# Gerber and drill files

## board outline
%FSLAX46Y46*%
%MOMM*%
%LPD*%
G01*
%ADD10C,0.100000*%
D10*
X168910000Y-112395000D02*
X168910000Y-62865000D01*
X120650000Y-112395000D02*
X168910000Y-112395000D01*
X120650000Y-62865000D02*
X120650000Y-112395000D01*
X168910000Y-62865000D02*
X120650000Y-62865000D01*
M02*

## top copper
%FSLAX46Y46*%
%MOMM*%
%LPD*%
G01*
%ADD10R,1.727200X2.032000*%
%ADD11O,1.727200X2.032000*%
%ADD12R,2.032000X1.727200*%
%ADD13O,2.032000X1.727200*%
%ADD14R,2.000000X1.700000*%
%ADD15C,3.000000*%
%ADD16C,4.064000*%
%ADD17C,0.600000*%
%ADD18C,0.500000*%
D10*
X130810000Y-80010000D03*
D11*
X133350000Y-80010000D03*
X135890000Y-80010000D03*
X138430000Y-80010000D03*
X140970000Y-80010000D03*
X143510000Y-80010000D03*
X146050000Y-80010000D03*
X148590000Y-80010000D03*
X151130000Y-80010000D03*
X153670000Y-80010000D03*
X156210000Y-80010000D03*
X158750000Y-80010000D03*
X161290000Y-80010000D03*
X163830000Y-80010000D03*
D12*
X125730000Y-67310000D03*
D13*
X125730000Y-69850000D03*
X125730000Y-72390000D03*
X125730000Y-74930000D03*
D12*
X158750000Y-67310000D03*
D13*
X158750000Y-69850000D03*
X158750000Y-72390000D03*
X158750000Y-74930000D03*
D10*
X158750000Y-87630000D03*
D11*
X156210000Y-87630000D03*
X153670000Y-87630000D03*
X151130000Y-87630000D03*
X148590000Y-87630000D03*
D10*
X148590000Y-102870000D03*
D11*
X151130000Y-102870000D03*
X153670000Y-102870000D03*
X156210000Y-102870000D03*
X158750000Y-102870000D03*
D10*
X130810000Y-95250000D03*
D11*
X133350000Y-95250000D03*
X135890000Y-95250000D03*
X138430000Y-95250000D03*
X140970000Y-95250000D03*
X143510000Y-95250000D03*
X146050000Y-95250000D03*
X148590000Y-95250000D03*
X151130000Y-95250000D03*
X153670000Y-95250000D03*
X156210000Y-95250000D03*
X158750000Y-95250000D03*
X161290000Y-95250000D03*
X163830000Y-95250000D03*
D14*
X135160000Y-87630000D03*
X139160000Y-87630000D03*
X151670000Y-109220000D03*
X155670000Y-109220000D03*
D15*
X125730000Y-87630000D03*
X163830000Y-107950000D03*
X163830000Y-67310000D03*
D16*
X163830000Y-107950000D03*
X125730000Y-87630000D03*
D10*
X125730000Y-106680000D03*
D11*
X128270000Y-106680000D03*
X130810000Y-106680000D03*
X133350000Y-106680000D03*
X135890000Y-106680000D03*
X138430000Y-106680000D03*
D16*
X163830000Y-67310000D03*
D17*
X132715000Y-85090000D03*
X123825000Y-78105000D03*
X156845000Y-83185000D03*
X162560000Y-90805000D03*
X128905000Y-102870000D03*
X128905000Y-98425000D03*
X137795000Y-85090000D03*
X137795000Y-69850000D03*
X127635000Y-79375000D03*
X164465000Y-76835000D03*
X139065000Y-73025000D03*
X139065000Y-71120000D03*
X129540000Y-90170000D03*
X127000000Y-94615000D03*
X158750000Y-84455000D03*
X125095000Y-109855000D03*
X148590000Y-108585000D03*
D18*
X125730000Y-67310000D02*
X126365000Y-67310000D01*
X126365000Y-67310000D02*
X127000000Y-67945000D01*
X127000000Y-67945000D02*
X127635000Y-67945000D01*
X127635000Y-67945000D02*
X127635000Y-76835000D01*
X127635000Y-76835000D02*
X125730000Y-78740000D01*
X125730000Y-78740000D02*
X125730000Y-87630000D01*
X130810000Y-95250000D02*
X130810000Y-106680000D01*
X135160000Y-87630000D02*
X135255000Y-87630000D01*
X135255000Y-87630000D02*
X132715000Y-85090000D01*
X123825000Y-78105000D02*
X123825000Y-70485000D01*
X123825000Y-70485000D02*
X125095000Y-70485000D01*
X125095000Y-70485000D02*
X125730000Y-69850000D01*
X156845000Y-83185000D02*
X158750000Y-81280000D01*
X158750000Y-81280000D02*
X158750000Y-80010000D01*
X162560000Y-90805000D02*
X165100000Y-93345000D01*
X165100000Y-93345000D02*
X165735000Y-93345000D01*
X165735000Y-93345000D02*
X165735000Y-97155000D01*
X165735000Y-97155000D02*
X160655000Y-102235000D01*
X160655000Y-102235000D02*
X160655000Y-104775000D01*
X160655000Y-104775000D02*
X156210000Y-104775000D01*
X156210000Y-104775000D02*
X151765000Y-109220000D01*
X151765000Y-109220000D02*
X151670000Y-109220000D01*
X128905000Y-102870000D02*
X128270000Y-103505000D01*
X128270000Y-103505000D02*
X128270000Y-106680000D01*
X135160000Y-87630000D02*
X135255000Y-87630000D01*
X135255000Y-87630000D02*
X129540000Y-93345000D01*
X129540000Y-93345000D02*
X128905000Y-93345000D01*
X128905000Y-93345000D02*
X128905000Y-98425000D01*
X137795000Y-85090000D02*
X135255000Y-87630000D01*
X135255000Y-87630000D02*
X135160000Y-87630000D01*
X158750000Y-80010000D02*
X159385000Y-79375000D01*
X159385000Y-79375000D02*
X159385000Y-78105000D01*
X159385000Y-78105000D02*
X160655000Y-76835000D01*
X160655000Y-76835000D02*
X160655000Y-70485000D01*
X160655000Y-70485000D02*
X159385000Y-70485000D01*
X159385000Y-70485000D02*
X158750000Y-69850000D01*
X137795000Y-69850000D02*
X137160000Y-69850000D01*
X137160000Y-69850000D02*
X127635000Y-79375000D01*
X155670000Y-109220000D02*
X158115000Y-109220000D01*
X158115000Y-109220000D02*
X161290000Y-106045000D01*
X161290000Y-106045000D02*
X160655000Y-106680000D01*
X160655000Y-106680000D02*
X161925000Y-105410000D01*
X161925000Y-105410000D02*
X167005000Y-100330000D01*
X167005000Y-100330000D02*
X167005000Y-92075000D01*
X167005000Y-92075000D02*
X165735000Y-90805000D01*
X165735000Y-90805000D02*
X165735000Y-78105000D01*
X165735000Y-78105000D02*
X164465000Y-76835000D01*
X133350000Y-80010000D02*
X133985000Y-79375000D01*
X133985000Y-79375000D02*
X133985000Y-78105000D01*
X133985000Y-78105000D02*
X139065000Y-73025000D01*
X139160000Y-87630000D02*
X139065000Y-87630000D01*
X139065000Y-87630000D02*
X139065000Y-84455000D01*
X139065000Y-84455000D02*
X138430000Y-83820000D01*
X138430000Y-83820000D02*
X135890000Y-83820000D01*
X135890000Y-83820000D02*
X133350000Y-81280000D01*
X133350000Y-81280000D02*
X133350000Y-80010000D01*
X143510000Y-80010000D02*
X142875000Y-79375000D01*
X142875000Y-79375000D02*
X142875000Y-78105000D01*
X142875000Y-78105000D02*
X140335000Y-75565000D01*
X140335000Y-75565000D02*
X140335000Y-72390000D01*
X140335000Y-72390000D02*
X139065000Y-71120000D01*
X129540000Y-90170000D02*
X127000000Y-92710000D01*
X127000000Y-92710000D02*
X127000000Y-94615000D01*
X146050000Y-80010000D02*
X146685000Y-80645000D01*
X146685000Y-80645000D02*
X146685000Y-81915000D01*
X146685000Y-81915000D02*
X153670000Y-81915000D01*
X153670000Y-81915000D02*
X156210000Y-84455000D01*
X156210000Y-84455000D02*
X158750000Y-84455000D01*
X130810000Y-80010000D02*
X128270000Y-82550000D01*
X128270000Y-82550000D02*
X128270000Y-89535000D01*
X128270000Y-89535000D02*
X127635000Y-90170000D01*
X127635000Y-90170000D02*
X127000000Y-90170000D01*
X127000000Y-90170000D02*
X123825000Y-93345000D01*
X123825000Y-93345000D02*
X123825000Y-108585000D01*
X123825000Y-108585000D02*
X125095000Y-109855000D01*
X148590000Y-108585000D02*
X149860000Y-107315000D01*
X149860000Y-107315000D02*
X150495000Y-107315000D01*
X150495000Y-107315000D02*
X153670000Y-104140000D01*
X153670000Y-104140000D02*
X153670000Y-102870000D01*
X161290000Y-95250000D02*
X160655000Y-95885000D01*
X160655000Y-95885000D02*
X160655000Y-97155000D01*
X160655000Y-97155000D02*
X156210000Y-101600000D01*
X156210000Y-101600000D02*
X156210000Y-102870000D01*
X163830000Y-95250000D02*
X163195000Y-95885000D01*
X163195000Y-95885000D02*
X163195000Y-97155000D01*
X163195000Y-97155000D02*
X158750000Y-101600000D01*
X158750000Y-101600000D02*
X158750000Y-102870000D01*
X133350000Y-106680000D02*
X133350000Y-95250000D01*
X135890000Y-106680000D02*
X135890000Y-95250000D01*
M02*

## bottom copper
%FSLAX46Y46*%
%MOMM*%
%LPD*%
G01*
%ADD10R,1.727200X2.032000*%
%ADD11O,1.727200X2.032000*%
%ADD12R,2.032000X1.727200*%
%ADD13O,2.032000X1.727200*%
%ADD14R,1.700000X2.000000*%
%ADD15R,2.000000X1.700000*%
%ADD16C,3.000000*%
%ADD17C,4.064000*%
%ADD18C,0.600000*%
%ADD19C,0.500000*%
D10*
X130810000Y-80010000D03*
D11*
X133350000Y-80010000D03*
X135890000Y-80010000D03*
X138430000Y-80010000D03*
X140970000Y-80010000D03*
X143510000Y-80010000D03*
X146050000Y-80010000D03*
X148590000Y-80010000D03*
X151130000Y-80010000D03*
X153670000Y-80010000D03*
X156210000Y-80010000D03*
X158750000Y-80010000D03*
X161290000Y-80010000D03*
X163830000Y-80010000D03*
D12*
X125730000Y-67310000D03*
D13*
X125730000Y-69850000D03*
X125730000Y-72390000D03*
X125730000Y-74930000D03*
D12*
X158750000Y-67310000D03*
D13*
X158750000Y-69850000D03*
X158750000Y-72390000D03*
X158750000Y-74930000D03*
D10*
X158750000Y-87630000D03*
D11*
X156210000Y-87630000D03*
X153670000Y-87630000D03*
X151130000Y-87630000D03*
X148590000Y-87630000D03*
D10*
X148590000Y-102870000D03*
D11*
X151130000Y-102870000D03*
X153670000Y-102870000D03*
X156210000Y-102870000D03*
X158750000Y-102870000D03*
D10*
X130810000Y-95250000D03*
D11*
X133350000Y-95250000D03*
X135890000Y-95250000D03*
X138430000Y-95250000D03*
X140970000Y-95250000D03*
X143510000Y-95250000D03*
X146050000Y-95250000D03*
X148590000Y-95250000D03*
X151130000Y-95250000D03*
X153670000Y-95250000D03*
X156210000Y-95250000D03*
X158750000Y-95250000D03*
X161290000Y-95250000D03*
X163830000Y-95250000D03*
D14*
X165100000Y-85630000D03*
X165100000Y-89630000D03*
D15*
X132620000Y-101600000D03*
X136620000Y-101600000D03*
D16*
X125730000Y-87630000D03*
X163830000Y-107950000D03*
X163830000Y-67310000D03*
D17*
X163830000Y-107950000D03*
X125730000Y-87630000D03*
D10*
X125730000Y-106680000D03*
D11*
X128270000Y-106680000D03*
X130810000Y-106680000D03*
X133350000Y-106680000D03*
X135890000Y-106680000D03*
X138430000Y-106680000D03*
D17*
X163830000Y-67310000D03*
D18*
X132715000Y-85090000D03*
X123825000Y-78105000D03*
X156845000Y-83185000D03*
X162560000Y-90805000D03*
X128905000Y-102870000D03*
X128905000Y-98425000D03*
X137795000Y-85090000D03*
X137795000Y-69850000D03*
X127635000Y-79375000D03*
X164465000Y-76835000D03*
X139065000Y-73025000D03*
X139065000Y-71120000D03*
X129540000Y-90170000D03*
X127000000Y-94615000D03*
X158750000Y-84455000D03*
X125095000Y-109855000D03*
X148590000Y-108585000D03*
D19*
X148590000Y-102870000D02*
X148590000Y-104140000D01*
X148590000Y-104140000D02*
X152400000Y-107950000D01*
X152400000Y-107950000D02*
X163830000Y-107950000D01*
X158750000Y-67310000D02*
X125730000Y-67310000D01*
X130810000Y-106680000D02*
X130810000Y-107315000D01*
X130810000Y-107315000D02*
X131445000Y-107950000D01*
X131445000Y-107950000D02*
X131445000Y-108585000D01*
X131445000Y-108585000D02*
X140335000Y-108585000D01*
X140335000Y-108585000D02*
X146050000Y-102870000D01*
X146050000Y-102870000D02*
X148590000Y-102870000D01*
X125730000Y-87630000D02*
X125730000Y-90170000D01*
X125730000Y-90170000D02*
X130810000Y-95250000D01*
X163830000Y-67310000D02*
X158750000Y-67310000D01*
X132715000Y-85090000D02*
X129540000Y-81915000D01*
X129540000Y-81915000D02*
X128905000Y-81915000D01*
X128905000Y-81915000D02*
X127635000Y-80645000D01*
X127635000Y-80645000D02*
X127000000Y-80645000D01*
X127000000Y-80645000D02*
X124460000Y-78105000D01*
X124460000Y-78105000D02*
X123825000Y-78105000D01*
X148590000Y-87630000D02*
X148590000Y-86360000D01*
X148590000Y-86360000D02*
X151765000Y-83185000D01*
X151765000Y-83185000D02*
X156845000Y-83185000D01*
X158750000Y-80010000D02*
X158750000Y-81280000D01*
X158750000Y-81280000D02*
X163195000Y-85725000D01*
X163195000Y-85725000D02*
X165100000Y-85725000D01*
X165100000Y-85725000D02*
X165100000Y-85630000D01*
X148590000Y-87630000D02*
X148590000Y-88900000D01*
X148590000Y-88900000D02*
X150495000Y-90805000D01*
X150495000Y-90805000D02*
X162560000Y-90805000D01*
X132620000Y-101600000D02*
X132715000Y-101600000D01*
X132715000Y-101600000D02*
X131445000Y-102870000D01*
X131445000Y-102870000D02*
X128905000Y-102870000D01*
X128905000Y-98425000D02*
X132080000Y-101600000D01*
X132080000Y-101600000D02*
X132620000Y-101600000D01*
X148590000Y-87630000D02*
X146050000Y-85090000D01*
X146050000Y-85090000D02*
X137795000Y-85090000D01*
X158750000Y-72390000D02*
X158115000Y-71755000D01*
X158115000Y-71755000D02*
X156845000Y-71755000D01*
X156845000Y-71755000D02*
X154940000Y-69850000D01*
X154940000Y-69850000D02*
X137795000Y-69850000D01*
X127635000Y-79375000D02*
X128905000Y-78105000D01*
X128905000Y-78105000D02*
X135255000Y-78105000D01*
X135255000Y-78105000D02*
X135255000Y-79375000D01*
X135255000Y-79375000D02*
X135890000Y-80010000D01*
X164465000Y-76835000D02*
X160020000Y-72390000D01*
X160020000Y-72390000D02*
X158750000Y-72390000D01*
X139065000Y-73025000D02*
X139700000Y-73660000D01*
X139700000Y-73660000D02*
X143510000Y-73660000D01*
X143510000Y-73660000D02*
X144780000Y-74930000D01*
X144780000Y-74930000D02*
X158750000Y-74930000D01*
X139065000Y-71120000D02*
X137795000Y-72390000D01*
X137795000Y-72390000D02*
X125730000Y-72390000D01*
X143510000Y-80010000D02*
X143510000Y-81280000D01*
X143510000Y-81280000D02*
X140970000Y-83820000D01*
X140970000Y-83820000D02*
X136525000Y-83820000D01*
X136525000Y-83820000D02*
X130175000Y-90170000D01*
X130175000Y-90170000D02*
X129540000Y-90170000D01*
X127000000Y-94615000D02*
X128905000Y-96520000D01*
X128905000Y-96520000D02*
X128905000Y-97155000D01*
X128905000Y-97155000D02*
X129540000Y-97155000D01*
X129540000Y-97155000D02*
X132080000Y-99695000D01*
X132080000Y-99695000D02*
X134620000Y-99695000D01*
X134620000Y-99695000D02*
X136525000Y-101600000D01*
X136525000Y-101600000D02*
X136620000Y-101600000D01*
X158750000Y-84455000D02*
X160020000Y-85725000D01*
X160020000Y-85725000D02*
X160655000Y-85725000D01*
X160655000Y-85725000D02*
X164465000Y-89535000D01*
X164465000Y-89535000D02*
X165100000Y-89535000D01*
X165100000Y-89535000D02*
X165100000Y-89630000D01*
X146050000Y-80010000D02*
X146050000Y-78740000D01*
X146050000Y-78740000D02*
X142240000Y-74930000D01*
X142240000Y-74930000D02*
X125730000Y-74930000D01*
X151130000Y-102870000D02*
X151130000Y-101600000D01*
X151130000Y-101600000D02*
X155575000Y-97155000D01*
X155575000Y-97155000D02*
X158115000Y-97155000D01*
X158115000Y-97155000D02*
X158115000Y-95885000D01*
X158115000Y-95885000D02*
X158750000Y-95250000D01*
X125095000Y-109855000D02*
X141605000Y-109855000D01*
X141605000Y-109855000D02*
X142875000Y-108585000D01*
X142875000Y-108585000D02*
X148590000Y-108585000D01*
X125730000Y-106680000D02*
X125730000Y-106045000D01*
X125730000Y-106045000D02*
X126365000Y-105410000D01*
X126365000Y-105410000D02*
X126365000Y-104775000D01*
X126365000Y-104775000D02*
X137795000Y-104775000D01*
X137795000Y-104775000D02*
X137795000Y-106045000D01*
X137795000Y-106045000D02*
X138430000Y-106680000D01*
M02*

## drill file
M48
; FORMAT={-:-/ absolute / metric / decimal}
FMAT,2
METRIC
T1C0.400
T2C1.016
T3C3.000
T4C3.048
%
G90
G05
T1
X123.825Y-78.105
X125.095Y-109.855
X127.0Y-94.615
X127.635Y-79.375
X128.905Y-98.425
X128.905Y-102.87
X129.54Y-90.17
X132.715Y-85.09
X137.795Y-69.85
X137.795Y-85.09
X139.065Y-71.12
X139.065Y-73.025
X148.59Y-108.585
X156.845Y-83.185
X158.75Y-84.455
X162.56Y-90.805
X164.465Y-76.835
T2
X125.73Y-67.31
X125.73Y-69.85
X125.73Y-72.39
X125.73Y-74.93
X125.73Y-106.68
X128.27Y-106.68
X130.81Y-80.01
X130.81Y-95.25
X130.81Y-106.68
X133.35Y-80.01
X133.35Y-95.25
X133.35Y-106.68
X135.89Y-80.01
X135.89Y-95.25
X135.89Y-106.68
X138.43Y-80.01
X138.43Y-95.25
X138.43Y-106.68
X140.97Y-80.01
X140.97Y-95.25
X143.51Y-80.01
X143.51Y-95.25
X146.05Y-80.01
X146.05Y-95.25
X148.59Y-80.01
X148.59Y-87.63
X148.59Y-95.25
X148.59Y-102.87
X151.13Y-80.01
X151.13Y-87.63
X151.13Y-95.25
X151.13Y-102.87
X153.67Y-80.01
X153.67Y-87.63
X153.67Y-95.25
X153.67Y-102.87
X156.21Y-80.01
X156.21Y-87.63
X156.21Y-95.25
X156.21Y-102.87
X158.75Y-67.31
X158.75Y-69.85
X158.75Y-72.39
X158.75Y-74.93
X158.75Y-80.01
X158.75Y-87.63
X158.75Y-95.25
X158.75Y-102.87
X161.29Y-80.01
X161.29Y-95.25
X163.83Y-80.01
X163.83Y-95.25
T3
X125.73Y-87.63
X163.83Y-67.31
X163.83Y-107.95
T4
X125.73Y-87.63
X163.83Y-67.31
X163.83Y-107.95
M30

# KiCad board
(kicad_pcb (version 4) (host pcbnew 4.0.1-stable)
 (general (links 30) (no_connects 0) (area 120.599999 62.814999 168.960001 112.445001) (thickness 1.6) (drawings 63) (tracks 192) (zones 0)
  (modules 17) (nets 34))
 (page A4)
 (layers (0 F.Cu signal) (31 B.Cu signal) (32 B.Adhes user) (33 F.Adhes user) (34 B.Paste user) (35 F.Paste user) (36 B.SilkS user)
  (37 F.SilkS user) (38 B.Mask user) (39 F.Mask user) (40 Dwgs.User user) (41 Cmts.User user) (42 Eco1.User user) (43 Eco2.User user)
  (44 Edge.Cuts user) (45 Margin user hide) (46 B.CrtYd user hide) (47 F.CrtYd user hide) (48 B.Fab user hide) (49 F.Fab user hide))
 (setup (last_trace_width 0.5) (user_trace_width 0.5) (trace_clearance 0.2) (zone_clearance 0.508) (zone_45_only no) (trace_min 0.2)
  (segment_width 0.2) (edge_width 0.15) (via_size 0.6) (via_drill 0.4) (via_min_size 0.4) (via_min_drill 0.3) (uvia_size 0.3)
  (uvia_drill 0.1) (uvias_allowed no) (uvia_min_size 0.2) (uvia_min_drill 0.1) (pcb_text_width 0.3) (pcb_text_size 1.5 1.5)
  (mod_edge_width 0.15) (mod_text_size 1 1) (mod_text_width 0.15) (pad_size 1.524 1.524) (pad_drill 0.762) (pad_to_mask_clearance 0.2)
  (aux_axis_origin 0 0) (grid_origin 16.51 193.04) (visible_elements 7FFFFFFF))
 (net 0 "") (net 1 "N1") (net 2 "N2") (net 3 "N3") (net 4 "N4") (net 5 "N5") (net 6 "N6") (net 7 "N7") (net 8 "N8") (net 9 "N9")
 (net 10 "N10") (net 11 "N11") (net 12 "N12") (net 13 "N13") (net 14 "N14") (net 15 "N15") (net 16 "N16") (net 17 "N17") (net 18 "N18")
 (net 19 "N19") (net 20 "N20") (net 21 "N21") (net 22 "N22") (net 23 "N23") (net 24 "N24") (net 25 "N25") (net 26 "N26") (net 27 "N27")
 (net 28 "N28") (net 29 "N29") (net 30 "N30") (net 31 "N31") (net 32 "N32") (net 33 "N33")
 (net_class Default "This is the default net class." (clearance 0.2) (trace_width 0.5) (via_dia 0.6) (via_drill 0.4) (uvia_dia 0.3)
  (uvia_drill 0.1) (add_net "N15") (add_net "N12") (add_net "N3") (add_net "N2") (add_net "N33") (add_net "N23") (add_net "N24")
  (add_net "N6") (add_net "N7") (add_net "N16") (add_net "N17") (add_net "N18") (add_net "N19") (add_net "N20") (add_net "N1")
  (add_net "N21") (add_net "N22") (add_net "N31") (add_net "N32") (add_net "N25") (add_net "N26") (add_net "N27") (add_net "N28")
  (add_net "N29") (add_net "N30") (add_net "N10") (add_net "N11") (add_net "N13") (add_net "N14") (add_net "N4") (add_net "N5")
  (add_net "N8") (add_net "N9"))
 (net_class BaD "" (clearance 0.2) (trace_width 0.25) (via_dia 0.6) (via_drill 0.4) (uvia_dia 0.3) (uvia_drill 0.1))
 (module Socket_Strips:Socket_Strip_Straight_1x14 (layer F.Cu) (at 130.81 80.01)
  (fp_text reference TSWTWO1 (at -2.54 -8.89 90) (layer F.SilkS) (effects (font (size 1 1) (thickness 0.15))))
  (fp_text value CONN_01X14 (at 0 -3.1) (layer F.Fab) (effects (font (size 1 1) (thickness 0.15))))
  (pad 1 thru_hole rect (at 0 0) (size 1.7272 2.032) (drill 1.016) (layers *.Cu *.Mask F.SilkS) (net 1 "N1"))
  (pad 2 thru_hole oval (at 2.54 0) (size 1.7272 2.032) (drill 1.016) (layers *.Cu *.Mask F.SilkS) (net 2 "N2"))
  (pad 3 thru_hole oval (at 5.08 0) (size 1.7272 2.032) (drill 1.016) (layers *.Cu *.Mask F.SilkS) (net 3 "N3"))
  (pad 4 thru_hole oval (at 7.62 0) (size 1.7272 2.032) (drill 1.016) (layers *.Cu *.Mask F.SilkS) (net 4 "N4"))
  (pad 5 thru_hole oval (at 10.16 0) (size 1.7272 2.032) (drill 1.016) (layers *.Cu *.Mask F.SilkS) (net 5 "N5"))
  (pad 6 thru_hole oval (at 12.7 0) (size 1.7272 2.032) (drill 1.016) (layers *.Cu *.Mask F.SilkS) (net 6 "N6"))
  (pad 7 thru_hole oval (at 15.24 0) (size 1.7272 2.032) (drill 1.016) (layers *.Cu *.Mask F.SilkS) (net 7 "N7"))
  (pad 8 thru_hole oval (at 17.78 0) (size 1.7272 2.032) (drill 1.016) (layers *.Cu *.Mask F.SilkS) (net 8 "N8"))
  (pad 9 thru_hole oval (at 20.32 0) (size 1.7272 2.032) (drill 1.016) (layers *.Cu *.Mask F.SilkS) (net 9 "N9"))
  (pad 10 thru_hole oval (at 22.86 0) (size 1.7272 2.032) (drill 1.016) (layers *.Cu *.Mask F.SilkS) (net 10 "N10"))
  (pad 11 thru_hole oval (at 25.4 0) (size 1.7272 2.032) (drill 1.016) (layers *.Cu *.Mask F.SilkS) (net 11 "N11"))
  (pad 12 thru_hole oval (at 27.94 0) (size 1.7272 2.032) (drill 1.016) (layers *.Cu *.Mask F.SilkS) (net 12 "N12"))
  (pad 13 thru_hole oval (at 30.48 0) (size 1.7272 2.032) (drill 1.016) (layers *.Cu *.Mask F.SilkS) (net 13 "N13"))
  (pad 14 thru_hole oval (at 33.02 0) (size 1.7272 2.032) (drill 1.016) (layers *.Cu *.Mask F.SilkS) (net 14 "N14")))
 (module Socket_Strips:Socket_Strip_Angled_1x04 (layer B.Cu) (at 125.73 67.31 270)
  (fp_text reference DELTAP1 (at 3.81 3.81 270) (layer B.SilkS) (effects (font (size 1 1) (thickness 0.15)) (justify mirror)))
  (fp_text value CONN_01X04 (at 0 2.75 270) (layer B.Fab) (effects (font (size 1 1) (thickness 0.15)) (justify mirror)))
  (pad 1 thru_hole rect (at 0 0 270) (size 1.7272 2.032) (drill 1.016) (layers *.Cu *.Mask B.SilkS) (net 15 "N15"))
  (pad 2 thru_hole oval (at 2.54 0 270) (size 1.7272 2.032) (drill 1.016) (layers *.Cu *.Mask B.SilkS) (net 12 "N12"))
  (pad 3 thru_hole oval (at 5.08 0 270) (size 1.7272 2.032) (drill 1.016) (layers *.Cu *.Mask B.SilkS) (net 6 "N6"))
  (pad 4 thru_hole oval (at 7.62 0 270) (size 1.7272 2.032) (drill 1.016) (layers *.Cu *.Mask B.SilkS) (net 7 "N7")))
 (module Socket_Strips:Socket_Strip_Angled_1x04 (layer F.Cu) (at 158.75 67.31 270)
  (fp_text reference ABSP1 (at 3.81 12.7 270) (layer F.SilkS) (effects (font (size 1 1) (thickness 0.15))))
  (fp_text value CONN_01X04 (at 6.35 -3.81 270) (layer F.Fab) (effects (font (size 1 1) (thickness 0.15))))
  (pad 1 thru_hole rect (at 0 0 270) (size 1.7272 2.032) (drill 1.016) (layers *.Cu *.Mask F.SilkS) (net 15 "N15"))
  (pad 2 thru_hole oval (at 2.54 0 270) (size 1.7272 2.032) (drill 1.016) (layers *.Cu *.Mask F.SilkS) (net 12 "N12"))
  (pad 3 thru_hole oval (at 5.08 0 270) (size 1.7272 2.032) (drill 1.016) (layers *.Cu *.Mask F.SilkS) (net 3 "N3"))
  (pad 4 thru_hole oval (at 7.62 0 270) (size 1.7272 2.032) (drill 1.016) (layers *.Cu *.Mask F.SilkS) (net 2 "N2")))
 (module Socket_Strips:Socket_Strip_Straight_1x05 (layer F.Cu) (at 158.75 87.63 180)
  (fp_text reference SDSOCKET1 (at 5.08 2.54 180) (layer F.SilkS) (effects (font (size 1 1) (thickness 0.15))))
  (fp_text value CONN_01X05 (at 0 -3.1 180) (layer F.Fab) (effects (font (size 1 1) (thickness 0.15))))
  (pad 1 thru_hole rect (at 0 0 180) (size 1.7272 2.032) (drill 1.016) (layers *.Cu *.Mask F.SilkS) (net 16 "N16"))
  (pad 2 thru_hole oval (at 2.54 0 180) (size 1.7272 2.032) (drill 1.016) (layers *.Cu *.Mask F.SilkS) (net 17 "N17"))
  (pad 3 thru_hole oval (at 5.08 0 180) (size 1.7272 2.032) (drill 1.016) (layers *.Cu *.Mask F.SilkS) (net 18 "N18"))
  (pad 4 thru_hole oval (at 7.62 0 180) (size 1.7272 2.032) (drill 1.016) (layers *.Cu *.Mask F.SilkS) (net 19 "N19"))
  (pad 5 thru_hole oval (at 10.16 0 180) (size 1.7272 2.032) (drill 1.016) (layers *.Cu *.Mask F.SilkS) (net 12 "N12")))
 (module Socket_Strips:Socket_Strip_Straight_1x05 (layer F.Cu) (at 148.59 102.87)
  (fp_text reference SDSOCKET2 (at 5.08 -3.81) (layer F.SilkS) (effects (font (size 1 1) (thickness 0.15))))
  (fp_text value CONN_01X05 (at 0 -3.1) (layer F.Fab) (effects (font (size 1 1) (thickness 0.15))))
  (pad 1 thru_hole rect (at 0 0) (size 1.7272 2.032) (drill 1.016) (layers *.Cu *.Mask F.SilkS) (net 15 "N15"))
  (pad 2 thru_hole oval (at 2.54 0) (size 1.7272 2.032) (drill 1.016) (layers *.Cu *.Mask F.SilkS) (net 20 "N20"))
  (pad 3 thru_hole oval (at 5.08 0) (size 1.7272 2.032) (drill 1.016) (layers *.Cu *.Mask F.SilkS) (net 1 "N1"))
  (pad 4 thru_hole oval (at 7.62 0) (size 1.7272 2.032) (drill 1.016) (layers *.Cu *.Mask F.SilkS) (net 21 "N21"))
  (pad 5 thru_hole oval (at 10.16 0) (size 1.7272 2.032) (drill 1.016) (layers *.Cu *.Mask F.SilkS) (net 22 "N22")))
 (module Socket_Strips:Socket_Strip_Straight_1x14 (layer F.Cu) (at 130.81 95.25)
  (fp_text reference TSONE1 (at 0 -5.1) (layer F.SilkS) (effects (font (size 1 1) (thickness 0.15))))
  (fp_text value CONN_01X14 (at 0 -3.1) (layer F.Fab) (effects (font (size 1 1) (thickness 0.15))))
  (pad 1 thru_hole rect (at 0 0) (size 1.7272 2.032) (drill 1.016) (layers *.Cu *.Mask F.SilkS) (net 15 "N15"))
  (pad 2 thru_hole oval (at 2.54 0) (size 1.7272 2.032) (drill 1.016) (layers *.Cu *.Mask F.SilkS) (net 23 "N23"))
  (pad 3 thru_hole oval (at 5.08 0) (size 1.7272 2.032) (drill 1.016) (layers *.Cu *.Mask F.SilkS) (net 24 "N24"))
  (pad 4 thru_hole oval (at 7.62 0) (size 1.7272 2.032) (drill 1.016) (layers *.Cu *.Mask F.SilkS) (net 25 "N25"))
  (pad 5 thru_hole oval (at 10.16 0) (size 1.7272 2.032) (drill 1.016) (layers *.Cu *.Mask F.SilkS) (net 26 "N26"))
  (pad 6 thru_hole oval (at 12.7 0) (size 1.7272 2.032) (drill 1.016) (layers *.Cu *.Mask F.SilkS) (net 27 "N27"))
  (pad 7 thru_hole oval (at 15.24 0) (size 1.7272 2.032) (drill 1.016) (layers *.Cu *.Mask F.SilkS) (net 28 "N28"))
  (pad 8 thru_hole oval (at 17.78 0) (size 1.7272 2.032) (drill 1.016) (layers *.Cu *.Mask F.SilkS) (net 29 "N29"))
  (pad 9 thru_hole oval (at 20.32 0) (size 1.7272 2.032) (drill 1.016) (layers *.Cu *.Mask F.SilkS) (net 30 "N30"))
  (pad 10 thru_hole oval (at 22.86 0) (size 1.7272 2.032) (drill 1.016) (layers *.Cu *.Mask F.SilkS) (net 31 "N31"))
  (pad 11 thru_hole oval (at 25.4 0) (size 1.7272 2.032) (drill 1.016) (layers *.Cu *.Mask F.SilkS) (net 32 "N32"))
  (pad 12 thru_hole oval (at 27.94 0) (size 1.7272 2.032) (drill 1.016) (layers *.Cu *.Mask F.SilkS) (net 20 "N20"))
  (pad 13 thru_hole oval (at 30.48 0) (size 1.7272 2.032) (drill 1.016) (layers *.Cu *.Mask F.SilkS) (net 21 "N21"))
  (pad 14 thru_hole oval (at 33.02 0) (size 1.7272 2.032) (drill 1.016) (layers *.Cu *.Mask F.SilkS) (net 22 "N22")))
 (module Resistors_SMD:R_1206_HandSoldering (layer F.Cu) (at 137.16 87.63)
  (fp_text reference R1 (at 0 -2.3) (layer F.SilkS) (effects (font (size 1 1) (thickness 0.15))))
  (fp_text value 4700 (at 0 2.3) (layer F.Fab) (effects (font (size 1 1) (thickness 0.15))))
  (pad 1 smd rect (at -2 0) (size 2 1.7) (layers F.Cu F.Paste F.Mask) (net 12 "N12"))
  (pad 2 smd rect (at 2 0) (size 2 1.7) (layers F.Cu F.Paste F.Mask) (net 2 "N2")))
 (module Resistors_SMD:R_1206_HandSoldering (layer F.Cu) (at 153.67 109.22)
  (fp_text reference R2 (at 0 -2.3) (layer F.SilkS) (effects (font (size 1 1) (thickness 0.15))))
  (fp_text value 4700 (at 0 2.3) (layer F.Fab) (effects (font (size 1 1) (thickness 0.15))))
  (pad 1 smd rect (at -2 0) (size 2 1.7) (layers F.Cu F.Paste F.Mask) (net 12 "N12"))
  (pad 2 smd rect (at 2 0) (size 2 1.7) (layers F.Cu F.Paste F.Mask) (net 3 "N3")))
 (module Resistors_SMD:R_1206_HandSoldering (layer B.Cu) (at 165.1 87.63 270)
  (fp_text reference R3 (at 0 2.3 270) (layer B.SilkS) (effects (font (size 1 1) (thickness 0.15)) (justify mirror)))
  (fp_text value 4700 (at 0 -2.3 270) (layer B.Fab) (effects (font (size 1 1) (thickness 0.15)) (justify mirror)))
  (pad 1 smd rect (at -2 0 270) (size 2 1.7) (layers B.Cu B.Paste B.Mask) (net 12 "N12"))
  (pad 2 smd rect (at 2 0 270) (size 2 1.7) (layers B.Cu B.Paste B.Mask) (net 7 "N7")))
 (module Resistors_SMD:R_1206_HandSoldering (layer B.Cu) (at 134.62 101.6)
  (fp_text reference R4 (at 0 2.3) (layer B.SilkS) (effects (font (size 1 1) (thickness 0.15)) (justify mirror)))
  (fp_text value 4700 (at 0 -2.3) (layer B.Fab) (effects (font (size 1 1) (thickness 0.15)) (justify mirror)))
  (pad 1 smd rect (at -2 0) (size 2 1.7) (layers B.Cu B.Paste B.Mask) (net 12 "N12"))
  (pad 2 smd rect (at 2 0) (size 2 1.7) (layers B.Cu B.Paste B.Mask) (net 6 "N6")))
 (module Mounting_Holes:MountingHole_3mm (layer F.Cu) (at 125.73 87.63)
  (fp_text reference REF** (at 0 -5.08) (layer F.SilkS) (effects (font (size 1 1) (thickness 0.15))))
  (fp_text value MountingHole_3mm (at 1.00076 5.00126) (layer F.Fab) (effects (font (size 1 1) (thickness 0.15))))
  (pad 1 thru_hole circle (at 0 0) (size 3 3) (drill 3) (layers)))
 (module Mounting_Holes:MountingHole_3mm (layer F.Cu) (at 163.83 107.95)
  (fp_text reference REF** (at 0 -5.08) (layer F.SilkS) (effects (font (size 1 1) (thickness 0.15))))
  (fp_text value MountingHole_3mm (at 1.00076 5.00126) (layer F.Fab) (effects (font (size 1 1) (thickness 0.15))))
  (pad 1 thru_hole circle (at 0 0) (size 3 3) (drill 3) (layers)))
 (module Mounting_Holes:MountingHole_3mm (layer F.Cu) (at 163.83 67.31)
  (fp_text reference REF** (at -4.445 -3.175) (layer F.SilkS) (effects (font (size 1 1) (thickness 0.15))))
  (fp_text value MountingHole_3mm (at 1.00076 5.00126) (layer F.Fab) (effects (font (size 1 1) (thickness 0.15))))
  (pad 1 thru_hole circle (at 0 0) (size 3 3) (drill 3) (layers)))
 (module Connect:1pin (layer F.Cu) (at 163.83 107.95)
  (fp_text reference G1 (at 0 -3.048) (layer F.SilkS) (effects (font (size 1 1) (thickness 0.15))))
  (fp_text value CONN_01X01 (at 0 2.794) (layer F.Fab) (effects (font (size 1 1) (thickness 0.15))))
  (pad 1 thru_hole circle (at 0 0) (size 4.064 4.064) (drill 3.048) (layers *.Cu *.Mask F.SilkS) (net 15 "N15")))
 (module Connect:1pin (layer F.Cu) (at 125.73 87.63)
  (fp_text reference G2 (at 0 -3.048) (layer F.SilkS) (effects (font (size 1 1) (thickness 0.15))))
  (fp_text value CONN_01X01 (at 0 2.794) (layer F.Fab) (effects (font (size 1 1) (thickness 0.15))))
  (pad 1 thru_hole circle (at 0 0) (size 4.064 4.064) (drill 3.048) (layers *.Cu *.Mask F.SilkS) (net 15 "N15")))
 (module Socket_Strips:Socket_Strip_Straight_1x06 (layer F.Cu) (at 125.73 106.68)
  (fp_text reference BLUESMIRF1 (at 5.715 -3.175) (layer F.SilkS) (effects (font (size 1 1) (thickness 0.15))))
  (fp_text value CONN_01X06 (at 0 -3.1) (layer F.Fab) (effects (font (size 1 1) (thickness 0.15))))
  (pad 1 thru_hole rect (at 0 0) (size 1.7272 2.032) (drill 1.016) (layers *.Cu *.Mask F.SilkS) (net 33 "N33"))
  (pad 2 thru_hole oval (at 2.54 0) (size 1.7272 2.032) (drill 1.016) (layers *.Cu *.Mask F.SilkS) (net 12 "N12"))
  (pad 3 thru_hole oval (at 5.08 0) (size 1.7272 2.032) (drill 1.016) (layers *.Cu *.Mask F.SilkS) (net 15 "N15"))
  (pad 4 thru_hole oval (at 7.62 0) (size 1.7272 2.032) (drill 1.016) (layers *.Cu *.Mask F.SilkS) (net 23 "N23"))
  (pad 5 thru_hole oval (at 10.16 0) (size 1.7272 2.032) (drill 1.016) (layers *.Cu *.Mask F.SilkS) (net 24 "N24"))
  (pad 6 thru_hole oval (at 12.7 0) (size 1.7272 2.032) (drill 1.016) (layers *.Cu *.Mask F.SilkS) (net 33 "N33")))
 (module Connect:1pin (layer F.Cu) (at 163.83 67.31)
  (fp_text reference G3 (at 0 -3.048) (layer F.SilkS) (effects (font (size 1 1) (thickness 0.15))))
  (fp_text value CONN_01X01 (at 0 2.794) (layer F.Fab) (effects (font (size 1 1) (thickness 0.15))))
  (pad 1 thru_hole circle (at 0 0) (size 4.064 4.064) (drill 3.048) (layers *.Cu *.Mask F.SilkS) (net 15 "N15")))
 (gr_line (start 168.91 112.395) (end 168.91 62.865) (layer Edge.Cuts) (width 0.1))
 (gr_line (start 120.65 112.395) (end 168.91 112.395) (layer Edge.Cuts) (width 0.1))
 (gr_line (start 120.65 62.865) (end 120.65 112.395) (layer Edge.Cuts) (width 0.1))
 (gr_line (start 168.91 62.865) (end 120.65 62.865) (layer Edge.Cuts) (width 0.1))
 (segment (start 148.59 102.87) (end 148.59 104.14) (width 0.5) (layer B.Cu) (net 15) (status 80000))
 (segment (start 148.59 104.14) (end 152.4 107.95) (width 0.5) (layer B.Cu) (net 15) (status 80000))
 (segment (start 152.4 107.95) (end 163.83 107.95) (width 0.5) (layer B.Cu) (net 15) (status 80000))
 (segment (start 158.75 67.31) (end 125.73 67.31) (width 0.5) (layer B.Cu) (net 15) (status 80000))
 (segment (start 130.81 106.68) (end 130.81 107.315) (width 0.5) (layer B.Cu) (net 15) (status 80000))
 (segment (start 130.81 107.315) (end 131.445 107.95) (width 0.5) (layer B.Cu) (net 15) (status 80000))
 (segment (start 131.445 107.95) (end 131.445 108.585) (width 0.5) (layer B.Cu) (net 15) (status 80000))
 (segment (start 131.445 108.585) (end 140.335 108.585) (width 0.5) (layer B.Cu) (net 15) (status 80000))
 (segment (start 140.335 108.585) (end 146.05 102.87) (width 0.5) (layer B.Cu) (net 15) (status 80000))
 (segment (start 146.05 102.87) (end 148.59 102.87) (width 0.5) (layer B.Cu) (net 15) (status 80000))
 (segment (start 125.73 87.63) (end 125.73 90.17) (width 0.5) (layer B.Cu) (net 15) (status 80000))
 (segment (start 125.73 90.17) (end 130.81 95.25) (width 0.5) (layer B.Cu) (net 15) (status 80000))
 (segment (start 125.73 67.31) (end 126.365 67.31) (width 0.5) (layer F.Cu) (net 15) (status 80000))
 (segment (start 126.365 67.31) (end 127 67.945) (width 0.5) (layer F.Cu) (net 15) (status 80000))
 (segment (start 127 67.945) (end 127.635 67.945) (width 0.5) (layer F.Cu) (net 15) (status 80000))
 (segment (start 127.635 67.945) (end 127.635 76.835) (width 0.5) (layer F.Cu) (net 15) (status 80000))
 (segment (start 127.635 76.835) (end 125.73 78.74) (width 0.5) (layer F.Cu) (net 15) (status 80000))
 (segment (start 125.73 78.74) (end 125.73 87.63) (width 0.5) (layer F.Cu) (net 15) (status 80000))
 (segment (start 130.81 95.25) (end 130.81 106.68) (width 0.5) (layer F.Cu) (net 15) (status 80000))
 (segment (start 163.83 67.31) (end 158.75 67.31) (width 0.5) (layer B.Cu) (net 15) (status 80000))
 (segment (start 135.16 87.63) (end 135.255 87.63) (width 0.5) (layer F.Cu) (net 12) (status 80000))
 (segment (start 135.255 87.63) (end 132.715 85.09) (width 0.5) (layer F.Cu) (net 12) (status 80000))
 (via (at 132.715 85.09) (size 0.6) (layers F.Cu B.Cu) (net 12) (status 80000))
 (segment (start 132.715 85.09) (end 129.54 81.915) (width 0.5) (layer B.Cu) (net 12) (status 80000))
 (segment (start 129.54 81.915) (end 128.905 81.915) (width 0.5) (layer B.Cu) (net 12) (status 80000))
 (segment (start 128.905 81.915) (end 127.635 80.645) (width 0.5) (layer B.Cu) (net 12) (status 80000))
 (segment (start 127.635 80.645) (end 127 80.645) (width 0.5) (layer B.Cu) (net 12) (status 80000))
 (segment (start 127 80.645) (end 124.46 78.105) (width 0.5) (layer B.Cu) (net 12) (status 80000))
 (segment (start 124.46 78.105) (end 123.825 78.105) (width 0.5) (layer B.Cu) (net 12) (status 80000))
 (via (at 123.825 78.105) (size 0.6) (layers F.Cu B.Cu) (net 12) (status 80000))
 (segment (start 123.825 78.105) (end 123.825 70.485) (width 0.5) (layer F.Cu) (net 12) (status 80000))
 (segment (start 123.825 70.485) (end 125.095 70.485) (width 0.5) (layer F.Cu) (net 12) (status 80000))
 (segment (start 125.095 70.485) (end 125.73 69.85) (width 0.5) (layer F.Cu) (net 12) (status 80000))
 (segment (start 148.59 87.63) (end 148.59 86.36) (width 0.5) (layer B.Cu) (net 12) (status 80000))
 (segment (start 148.59 86.36) (end 151.765 83.185) (width 0.5) (layer B.Cu) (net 12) (status 80000))
 (segment (start 151.765 83.185) (end 156.845 83.185) (width 0.5) (layer B.Cu) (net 12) (status 80000))
 (via (at 156.845 83.185) (size 0.6) (layers F.Cu B.Cu) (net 12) (status 80000))
 (segment (start 156.845 83.185) (end 158.75 81.28) (width 0.5) (layer F.Cu) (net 12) (status 80000))
 (segment (start 158.75 81.28) (end 158.75 80.01) (width 0.5) (layer F.Cu) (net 12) (status 80000))
 (segment (start 158.75 80.01) (end 158.75 81.28) (width 0.5) (layer B.Cu) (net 12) (status 80000))
 (segment (start 158.75 81.28) (end 163.195 85.725) (width 0.5) (layer B.Cu) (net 12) (status 80000))
 (segment (start 163.195 85.725) (end 165.1 85.725) (width 0.5) (layer B.Cu) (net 12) (status 80000))
 (segment (start 165.1 85.725) (end 165.1 85.63) (width 0.5) (layer B.Cu) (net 12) (status 80000))
 (segment (start 148.59 87.63) (end 148.59 88.9) (width 0.5) (layer B.Cu) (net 12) (status 80000))
 (segment (start 148.59 88.9) (end 150.495 90.805) (width 0.5) (layer B.Cu) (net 12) (status 80000))
 (segment (start 150.495 90.805) (end 162.56 90.805) (width 0.5) (layer B.Cu) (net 12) (status 80000))
 (via (at 162.56 90.805) (size 0.6) (layers F.Cu B.Cu) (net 12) (status 80000))
 (segment (start 162.56 90.805) (end 165.1 93.345) (width 0.5) (layer F.Cu) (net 12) (status 80000))
 (segment (start 165.1 93.345) (end 165.735 93.345) (width 0.5) (layer F.Cu) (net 12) (status 80000))
 (segment (start 165.735 93.345) (end 165.735 97.155) (width 0.5) (layer F.Cu) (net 12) (status 80000))
 (segment (start 165.735 97.155) (end 160.655 102.235) (width 0.5) (layer F.Cu) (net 12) (status 80000))
 (segment (start 160.655 102.235) (end 160.655 104.775) (width 0.5) (layer F.Cu) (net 12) (status 80000))
 (segment (start 160.655 104.775) (end 156.21 104.775) (width 0.5) (layer F.Cu) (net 12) (status 80000))
 (segment (start 156.21 104.775) (end 151.765 109.22) (width 0.5) (layer F.Cu) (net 12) (status 80000))
 (segment (start 151.765 109.22) (end 151.67 109.22) (width 0.5) (layer F.Cu) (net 12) (status 80000))
 (segment (start 132.62 101.6) (end 132.715 101.6) (width 0.5) (layer B.Cu) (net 12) (status 80000))
 (segment (start 132.715 101.6) (end 131.445 102.87) (width 0.5) (layer B.Cu) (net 12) (status 80000))
 (segment (start 131.445 102.87) (end 128.905 102.87) (width 0.5) (layer B.Cu) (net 12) (status 80000))
 (via (at 128.905 102.87) (size 0.6) (layers F.Cu B.Cu) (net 12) (status 80000))
 (segment (start 128.905 102.87) (end 128.27 103.505) (width 0.5) (layer F.Cu) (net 12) (status 80000))
 (segment (start 128.27 103.505) (end 128.27 106.68) (width 0.5) (layer F.Cu) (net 12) (status 80000))
 (segment (start 135.16 87.63) (end 135.255 87.63) (width 0.5) (layer F.Cu) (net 12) (status 80000))
 (segment (start 135.255 87.63) (end 129.54 93.345) (width 0.5) (layer F.Cu) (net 12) (status 80000))
 (segment (start 129.54 93.345) (end 128.905 93.345) (width 0.5) (layer F.Cu) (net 12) (status 80000))
 (segment (start 128.905 93.345) (end 128.905 98.425) (width 0.5) (layer F.Cu) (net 12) (status 80000))
 (via (at 128.905 98.425) (size 0.6) (layers F.Cu B.Cu) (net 12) (status 80000))
 (segment (start 128.905 98.425) (end 132.08 101.6) (width 0.5) (layer B.Cu) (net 12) (status 80000))
 (segment (start 132.08 101.6) (end 132.62 101.6) (width 0.5) (layer B.Cu) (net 12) (status 80000))
 (segment (start 148.59 87.63) (end 146.05 85.09) (width 0.5) (layer B.Cu) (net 12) (status 80000))
 (segment (start 146.05 85.09) (end 137.795 85.09) (width 0.5) (layer B.Cu) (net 12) (status 80000))
 (via (at 137.795 85.09) (size 0.6) (layers F.Cu B.Cu) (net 12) (status 80000))
 (segment (start 137.795 85.09) (end 135.255 87.63) (width 0.5) (layer F.Cu) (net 12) (status 80000))
 (segment (start 135.255 87.63) (end 135.16 87.63) (width 0.5) (layer F.Cu) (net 12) (status 80000))
 (segment (start 158.75 80.01) (end 159.385 79.375) (width 0.5) (layer F.Cu) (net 12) (status 80000))
 (segment (start 159.385 79.375) (end 159.385 78.105) (width 0.5) (layer F.Cu) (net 12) (status 80000))
 (segment (start 159.385 78.105) (end 160.655 76.835) (width 0.5) (layer F.Cu) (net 12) (status 80000))
 (segment (start 160.655 76.835) (end 160.655 70.485) (width 0.5) (layer F.Cu) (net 12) (status 80000))
 (segment (start 160.655 70.485) (end 159.385 70.485) (width 0.5) (layer F.Cu) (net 12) (status 80000))
 (segment (start 159.385 70.485) (end 158.75 69.85) (width 0.5) (layer F.Cu) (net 12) (status 80000))
 (segment (start 158.75 72.39) (end 158.115 71.755) (width 0.5) (layer B.Cu) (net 3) (status 80000))
 (segment (start 158.115 71.755) (end 156.845 71.755) (width 0.5) (layer B.Cu) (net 3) (status 80000))
 (segment (start 156.845 71.755) (end 154.94 69.85) (width 0.5) (layer B.Cu) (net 3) (status 80000))
 (segment (start 154.94 69.85) (end 137.795 69.85) (width 0.5) (layer B.Cu) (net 3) (status 80000))
 (via (at 137.795 69.85) (size 0.6) (layers F.Cu B.Cu) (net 3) (status 80000))
 (segment (start 137.795 69.85) (end 137.16 69.85) (width 0.5) (layer F.Cu) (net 3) (status 80000))
 (segment (start 137.16 69.85) (end 127.635 79.375) (width 0.5) (layer F.Cu) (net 3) (status 80000))
 (via (at 127.635 79.375) (size 0.6) (layers F.Cu B.Cu) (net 3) (status 80000))
 (segment (start 127.635 79.375) (end 128.905 78.105) (width 0.5) (layer B.Cu) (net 3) (status 80000))
 (segment (start 128.905 78.105) (end 135.255 78.105) (width 0.5) (layer B.Cu) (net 3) (status 80000))
 (segment (start 135.255 78.105) (end 135.255 79.375) (width 0.5) (layer B.Cu) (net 3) (status 80000))
 (segment (start 135.255 79.375) (end 135.89 80.01) (width 0.5) (layer B.Cu) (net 3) (status 80000))
 (segment (start 155.67 109.22) (end 158.115 109.22) (width 0.5) (layer F.Cu) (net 3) (status 80000))
 (segment (start 158.115 109.22) (end 161.29 106.045) (width 0.5) (layer F.Cu) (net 3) (status 80000))
 (segment (start 161.29 106.045) (end 160.655 106.68) (width 0.5) (layer F.Cu) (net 3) (status 80000))
 (segment (start 160.655 106.68) (end 161.925 105.41) (width 0.5) (layer F.Cu) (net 3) (status 80000))
 (segment (start 161.925 105.41) (end 167.005 100.33) (width 0.5) (layer F.Cu) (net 3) (status 80000))
 (segment (start 167.005 100.33) (end 167.005 92.075) (width 0.5) (layer F.Cu) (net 3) (status 80000))
 (segment (start 167.005 92.075) (end 165.735 90.805) (width 0.5) (layer F.Cu) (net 3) (status 80000))
 (segment (start 165.735 90.805) (end 165.735 78.105) (width 0.5) (layer F.Cu) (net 3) (status 80000))
 (segment (start 165.735 78.105) (end 164.465 76.835) (width 0.5) (layer F.Cu) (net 3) (status 80000))
 (via (at 164.465 76.835) (size 0.6) (layers F.Cu B.Cu) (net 3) (status 80000))
 (segment (start 164.465 76.835) (end 160.02 72.39) (width 0.5) (layer B.Cu) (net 3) (status 80000))
 (segment (start 160.02 72.39) (end 158.75 72.39) (width 0.5) (layer B.Cu) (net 3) (status 80000))
 (segment (start 133.35 80.01) (end 133.985 79.375) (width 0.5) (layer F.Cu) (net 2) (status 80000))
 (segment (start 133.985 79.375) (end 133.985 78.105) (width 0.5) (layer F.Cu) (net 2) (status 80000))
 (segment (start 133.985 78.105) (end 139.065 73.025) (width 0.5) (layer F.Cu) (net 2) (status 80000))
 (via (at 139.065 73.025) (size 0.6) (layers F.Cu B.Cu) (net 2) (status 80000))
 (segment (start 139.065 73.025) (end 139.7 73.66) (width 0.5) (layer B.Cu) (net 2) (status 80000))
 (segment (start 139.7 73.66) (end 143.51 73.66) (width 0.5) (layer B.Cu) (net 2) (status 80000))
 (segment (start 143.51 73.66) (end 144.78 74.93) (width 0.5) (layer B.Cu) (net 2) (status 80000))
 (segment (start 144.78 74.93) (end 158.75 74.93) (width 0.5) (layer B.Cu) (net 2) (status 80000))
 (segment (start 139.16 87.63) (end 139.065 87.63) (width 0.5) (layer F.Cu) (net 2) (status 80000))
 (segment (start 139.065 87.63) (end 139.065 84.455) (width 0.5) (layer F.Cu) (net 2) (status 80000))
 (segment (start 139.065 84.455) (end 138.43 83.82) (width 0.5) (layer F.Cu) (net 2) (status 80000))
 (segment (start 138.43 83.82) (end 135.89 83.82) (width 0.5) (layer F.Cu) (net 2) (status 80000))
 (segment (start 135.89 83.82) (end 133.35 81.28) (width 0.5) (layer F.Cu) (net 2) (status 80000))
 (segment (start 133.35 81.28) (end 133.35 80.01) (width 0.5) (layer F.Cu) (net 2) (status 80000))
 (segment (start 143.51 80.01) (end 142.875 79.375) (width 0.5) (layer F.Cu) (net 6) (status 80000))
 (segment (start 142.875 79.375) (end 142.875 78.105) (width 0.5) (layer F.Cu) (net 6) (status 80000))
 (segment (start 142.875 78.105) (end 140.335 75.565) (width 0.5) (layer F.Cu) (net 6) (status 80000))
 (segment (start 140.335 75.565) (end 140.335 72.39) (width 0.5) (layer F.Cu) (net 6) (status 80000))
 (segment (start 140.335 72.39) (end 139.065 71.12) (width 0.5) (layer F.Cu) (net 6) (status 80000))
 (via (at 139.065 71.12) (size 0.6) (layers F.Cu B.Cu) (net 6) (status 80000))
 (segment (start 139.065 71.12) (end 137.795 72.39) (width 0.5) (layer B.Cu) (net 6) (status 80000))
 (segment (start 137.795 72.39) (end 125.73 72.39) (width 0.5) (layer B.Cu) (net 6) (status 80000))
 (segment (start 143.51 80.01) (end 143.51 81.28) (width 0.5) (layer B.Cu) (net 6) (status 80000))
 (segment (start 143.51 81.28) (end 140.97 83.82) (width 0.5) (layer B.Cu) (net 6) (status 80000))
 (segment (start 140.97 83.82) (end 136.525 83.82) (width 0.5) (layer B.Cu) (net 6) (status 80000))
 (segment (start 136.525 83.82) (end 130.175 90.17) (width 0.5) (layer B.Cu) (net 6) (status 80000))
 (segment (start 130.175 90.17) (end 129.54 90.17) (width 0.5) (layer B.Cu) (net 6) (status 80000))
 (via (at 129.54 90.17) (size 0.6) (layers F.Cu B.Cu) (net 6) (status 80000))
 (segment (start 129.54 90.17) (end 127 92.71) (width 0.5) (layer F.Cu) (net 6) (status 80000))
 (segment (start 127 92.71) (end 127 94.615) (width 0.5) (layer F.Cu) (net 6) (status 80000))
 (via (at 127 94.615) (size 0.6) (layers F.Cu B.Cu) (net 6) (status 80000))
 (segment (start 127 94.615) (end 128.905 96.52) (width 0.5) (layer B.Cu) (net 6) (status 80000))
 (segment (start 128.905 96.52) (end 128.905 97.155) (width 0.5) (layer B.Cu) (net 6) (status 80000))
 (segment (start 128.905 97.155) (end 129.54 97.155) (width 0.5) (layer B.Cu) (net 6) (status 80000))
 (segment (start 129.54 97.155) (end 132.08 99.695) (width 0.5) (layer B.Cu) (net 6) (status 80000))
 (segment (start 132.08 99.695) (end 134.62 99.695) (width 0.5) (layer B.Cu) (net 6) (status 80000))
 (segment (start 134.62 99.695) (end 136.525 101.6) (width 0.5) (layer B.Cu) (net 6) (status 80000))
 (segment (start 136.525 101.6) (end 136.62 101.6) (width 0.5) (layer B.Cu) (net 6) (status 80000))
 (segment (start 146.05 80.01) (end 146.685 80.645) (width 0.5) (layer F.Cu) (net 7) (status 80000))
 (segment (start 146.685 80.645) (end 146.685 81.915) (width 0.5) (layer F.Cu) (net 7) (status 80000))
 (segment (start 146.685 81.915) (end 153.67 81.915) (width 0.5) (layer F.Cu) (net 7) (status 80000))
 (segment (start 153.67 81.915) (end 156.21 84.455) (width 0.5) (layer F.Cu) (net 7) (status 80000))
 (segment (start 156.21 84.455) (end 158.75 84.455) (width 0.5) (layer F.Cu) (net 7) (status 80000))
 (via (at 158.75 84.455) (size 0.6) (layers F.Cu B.Cu) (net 7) (status 80000))
 (segment (start 158.75 84.455) (end 160.02 85.725) (width 0.5) (layer B.Cu) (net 7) (status 80000))
 (segment (start 160.02 85.725) (end 160.655 85.725) (width 0.5) (layer B.Cu) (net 7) (status 80000))
 (segment (start 160.655 85.725) (end 164.465 89.535) (width 0.5) (layer B.Cu) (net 7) (status 80000))
 (segment (start 164.465 89.535) (end 165.1 89.535) (width 0.5) (layer B.Cu) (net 7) (status 80000))
 (segment (start 165.1 89.535) (end 165.1 89.63) (width 0.5) (layer B.Cu) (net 7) (status 80000))
 (segment (start 146.05 80.01) (end 146.05 78.74) (width 0.5) (layer B.Cu) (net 7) (status 80000))
 (segment (start 146.05 78.74) (end 142.24 74.93) (width 0.5) (layer B.Cu) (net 7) (status 80000))
 (segment (start 142.24 74.93) (end 125.73 74.93) (width 0.5) (layer B.Cu) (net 7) (status 80000))
 (segment (start 151.13 102.87) (end 151.13 101.6) (width 0.5) (layer B.Cu) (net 20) (status 80000))
 (segment (start 151.13 101.6) (end 155.575 97.155) (width 0.5) (layer B.Cu) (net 20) (status 80000))
 (segment (start 155.575 97.155) (end 158.115 97.155) (width 0.5) (layer B.Cu) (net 20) (status 80000))
 (segment (start 158.115 97.155) (end 158.115 95.885) (width 0.5) (layer B.Cu) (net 20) (status 80000))
 (segment (start 158.115 95.885) (end 158.75 95.25) (width 0.5) (layer B.Cu) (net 20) (status 80000))
 (segment (start 130.81 80.01) (end 128.27 82.55) (width 0.5) (layer F.Cu) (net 1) (status 80000))
 (segment (start 128.27 82.55) (end 128.27 89.535) (width 0.5) (layer F.Cu) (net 1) (status 80000))
 (segment (start 128.27 89.535) (end 127.635 90.17) (width 0.5) (layer F.Cu) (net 1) (status 80000))
 (segment (start 127.635 90.17) (end 127 90.17) (width 0.5) (layer F.Cu) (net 1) (status 80000))
 (segment (start 127 90.17) (end 123.825 93.345) (width 0.5) (layer F.Cu) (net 1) (status 80000))
 (segment (start 123.825 93.345) (end 123.825 108.585) (width 0.5) (layer F.Cu) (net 1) (status 80000))
 (segment (start 123.825 108.585) (end 125.095 109.855) (width 0.5) (layer F.Cu) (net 1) (status 80000))
 (via (at 125.095 109.855) (size 0.6) (layers F.Cu B.Cu) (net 1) (status 80000))
 (segment (start 125.095 109.855) (end 141.605 109.855) (width 0.5) (layer B.Cu) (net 1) (status 80000))
 (segment (start 141.605 109.855) (end 142.875 108.585) (width 0.5) (layer B.Cu) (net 1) (status 80000))
 (segment (start 142.875 108.585) (end 148.59 108.585) (width 0.5) (layer B.Cu) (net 1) (status 80000))
 (via (at 148.59 108.585) (size 0.6) (layers F.Cu B.Cu) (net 1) (status 80000))
 (segment (start 148.59 108.585) (end 149.86 107.315) (width 0.5) (layer F.Cu) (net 1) (status 80000))
 (segment (start 149.86 107.315) (end 150.495 107.315) (width 0.5) (layer F.Cu) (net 1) (status 80000))
 (segment (start 150.495 107.315) (end 153.67 104.14) (width 0.5) (layer F.Cu) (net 1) (status 80000))
 (segment (start 153.67 104.14) (end 153.67 102.87) (width 0.5) (layer F.Cu) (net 1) (status 80000))
 (segment (start 161.29 95.25) (end 160.655 95.885) (width 0.5) (layer F.Cu) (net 21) (status 80000))
 (segment (start 160.655 95.885) (end 160.655 97.155) (width 0.5) (layer F.Cu) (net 21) (status 80000))
 (segment (start 160.655 97.155) (end 156.21 101.6) (width 0.5) (layer F.Cu) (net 21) (status 80000))
 (segment (start 156.21 101.6) (end 156.21 102.87) (width 0.5) (layer F.Cu) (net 21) (status 80000))
 (segment (start 163.83 95.25) (end 163.195 95.885) (width 0.5) (layer F.Cu) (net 22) (status 80000))
 (segment (start 163.195 95.885) (end 163.195 97.155) (width 0.5) (layer F.Cu) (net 22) (status 80000))
 (segment (start 163.195 97.155) (end 158.75 101.6) (width 0.5) (layer F.Cu) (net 22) (status 80000))
 (segment (start 158.75 101.6) (end 158.75 102.87) (width 0.5) (layer F.Cu) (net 22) (status 80000))
 (segment (start 125.73 106.68) (end 125.73 106.045) (width 0.5) (layer B.Cu) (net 33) (status 80000))
 (segment (start 125.73 106.045) (end 126.365 105.41) (width 0.5) (layer B.Cu) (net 33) (status 80000))
 (segment (start 126.365 105.41) (end 126.365 104.775) (width 0.5) (layer B.Cu) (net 33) (status 80000))
 (segment (start 126.365 104.775) (end 137.795 104.775) (width 0.5) (layer B.Cu) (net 33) (status 80000))
 (segment (start 137.795 104.775) (end 137.795 106.045) (width 0.5) (layer B.Cu) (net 33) (status 80000))
 (segment (start 137.795 106.045) (end 138.43 106.68) (width 0.5) (layer B.Cu) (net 33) (status 80000))
 (segment (start 133.35 106.68) (end 133.35 95.25) (width 0.5) (layer F.Cu) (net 23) (status 80000))
 (segment (start 135.89 106.68) (end 135.89 95.25) (width 0.5) (layer F.Cu) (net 24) (status 80000)))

